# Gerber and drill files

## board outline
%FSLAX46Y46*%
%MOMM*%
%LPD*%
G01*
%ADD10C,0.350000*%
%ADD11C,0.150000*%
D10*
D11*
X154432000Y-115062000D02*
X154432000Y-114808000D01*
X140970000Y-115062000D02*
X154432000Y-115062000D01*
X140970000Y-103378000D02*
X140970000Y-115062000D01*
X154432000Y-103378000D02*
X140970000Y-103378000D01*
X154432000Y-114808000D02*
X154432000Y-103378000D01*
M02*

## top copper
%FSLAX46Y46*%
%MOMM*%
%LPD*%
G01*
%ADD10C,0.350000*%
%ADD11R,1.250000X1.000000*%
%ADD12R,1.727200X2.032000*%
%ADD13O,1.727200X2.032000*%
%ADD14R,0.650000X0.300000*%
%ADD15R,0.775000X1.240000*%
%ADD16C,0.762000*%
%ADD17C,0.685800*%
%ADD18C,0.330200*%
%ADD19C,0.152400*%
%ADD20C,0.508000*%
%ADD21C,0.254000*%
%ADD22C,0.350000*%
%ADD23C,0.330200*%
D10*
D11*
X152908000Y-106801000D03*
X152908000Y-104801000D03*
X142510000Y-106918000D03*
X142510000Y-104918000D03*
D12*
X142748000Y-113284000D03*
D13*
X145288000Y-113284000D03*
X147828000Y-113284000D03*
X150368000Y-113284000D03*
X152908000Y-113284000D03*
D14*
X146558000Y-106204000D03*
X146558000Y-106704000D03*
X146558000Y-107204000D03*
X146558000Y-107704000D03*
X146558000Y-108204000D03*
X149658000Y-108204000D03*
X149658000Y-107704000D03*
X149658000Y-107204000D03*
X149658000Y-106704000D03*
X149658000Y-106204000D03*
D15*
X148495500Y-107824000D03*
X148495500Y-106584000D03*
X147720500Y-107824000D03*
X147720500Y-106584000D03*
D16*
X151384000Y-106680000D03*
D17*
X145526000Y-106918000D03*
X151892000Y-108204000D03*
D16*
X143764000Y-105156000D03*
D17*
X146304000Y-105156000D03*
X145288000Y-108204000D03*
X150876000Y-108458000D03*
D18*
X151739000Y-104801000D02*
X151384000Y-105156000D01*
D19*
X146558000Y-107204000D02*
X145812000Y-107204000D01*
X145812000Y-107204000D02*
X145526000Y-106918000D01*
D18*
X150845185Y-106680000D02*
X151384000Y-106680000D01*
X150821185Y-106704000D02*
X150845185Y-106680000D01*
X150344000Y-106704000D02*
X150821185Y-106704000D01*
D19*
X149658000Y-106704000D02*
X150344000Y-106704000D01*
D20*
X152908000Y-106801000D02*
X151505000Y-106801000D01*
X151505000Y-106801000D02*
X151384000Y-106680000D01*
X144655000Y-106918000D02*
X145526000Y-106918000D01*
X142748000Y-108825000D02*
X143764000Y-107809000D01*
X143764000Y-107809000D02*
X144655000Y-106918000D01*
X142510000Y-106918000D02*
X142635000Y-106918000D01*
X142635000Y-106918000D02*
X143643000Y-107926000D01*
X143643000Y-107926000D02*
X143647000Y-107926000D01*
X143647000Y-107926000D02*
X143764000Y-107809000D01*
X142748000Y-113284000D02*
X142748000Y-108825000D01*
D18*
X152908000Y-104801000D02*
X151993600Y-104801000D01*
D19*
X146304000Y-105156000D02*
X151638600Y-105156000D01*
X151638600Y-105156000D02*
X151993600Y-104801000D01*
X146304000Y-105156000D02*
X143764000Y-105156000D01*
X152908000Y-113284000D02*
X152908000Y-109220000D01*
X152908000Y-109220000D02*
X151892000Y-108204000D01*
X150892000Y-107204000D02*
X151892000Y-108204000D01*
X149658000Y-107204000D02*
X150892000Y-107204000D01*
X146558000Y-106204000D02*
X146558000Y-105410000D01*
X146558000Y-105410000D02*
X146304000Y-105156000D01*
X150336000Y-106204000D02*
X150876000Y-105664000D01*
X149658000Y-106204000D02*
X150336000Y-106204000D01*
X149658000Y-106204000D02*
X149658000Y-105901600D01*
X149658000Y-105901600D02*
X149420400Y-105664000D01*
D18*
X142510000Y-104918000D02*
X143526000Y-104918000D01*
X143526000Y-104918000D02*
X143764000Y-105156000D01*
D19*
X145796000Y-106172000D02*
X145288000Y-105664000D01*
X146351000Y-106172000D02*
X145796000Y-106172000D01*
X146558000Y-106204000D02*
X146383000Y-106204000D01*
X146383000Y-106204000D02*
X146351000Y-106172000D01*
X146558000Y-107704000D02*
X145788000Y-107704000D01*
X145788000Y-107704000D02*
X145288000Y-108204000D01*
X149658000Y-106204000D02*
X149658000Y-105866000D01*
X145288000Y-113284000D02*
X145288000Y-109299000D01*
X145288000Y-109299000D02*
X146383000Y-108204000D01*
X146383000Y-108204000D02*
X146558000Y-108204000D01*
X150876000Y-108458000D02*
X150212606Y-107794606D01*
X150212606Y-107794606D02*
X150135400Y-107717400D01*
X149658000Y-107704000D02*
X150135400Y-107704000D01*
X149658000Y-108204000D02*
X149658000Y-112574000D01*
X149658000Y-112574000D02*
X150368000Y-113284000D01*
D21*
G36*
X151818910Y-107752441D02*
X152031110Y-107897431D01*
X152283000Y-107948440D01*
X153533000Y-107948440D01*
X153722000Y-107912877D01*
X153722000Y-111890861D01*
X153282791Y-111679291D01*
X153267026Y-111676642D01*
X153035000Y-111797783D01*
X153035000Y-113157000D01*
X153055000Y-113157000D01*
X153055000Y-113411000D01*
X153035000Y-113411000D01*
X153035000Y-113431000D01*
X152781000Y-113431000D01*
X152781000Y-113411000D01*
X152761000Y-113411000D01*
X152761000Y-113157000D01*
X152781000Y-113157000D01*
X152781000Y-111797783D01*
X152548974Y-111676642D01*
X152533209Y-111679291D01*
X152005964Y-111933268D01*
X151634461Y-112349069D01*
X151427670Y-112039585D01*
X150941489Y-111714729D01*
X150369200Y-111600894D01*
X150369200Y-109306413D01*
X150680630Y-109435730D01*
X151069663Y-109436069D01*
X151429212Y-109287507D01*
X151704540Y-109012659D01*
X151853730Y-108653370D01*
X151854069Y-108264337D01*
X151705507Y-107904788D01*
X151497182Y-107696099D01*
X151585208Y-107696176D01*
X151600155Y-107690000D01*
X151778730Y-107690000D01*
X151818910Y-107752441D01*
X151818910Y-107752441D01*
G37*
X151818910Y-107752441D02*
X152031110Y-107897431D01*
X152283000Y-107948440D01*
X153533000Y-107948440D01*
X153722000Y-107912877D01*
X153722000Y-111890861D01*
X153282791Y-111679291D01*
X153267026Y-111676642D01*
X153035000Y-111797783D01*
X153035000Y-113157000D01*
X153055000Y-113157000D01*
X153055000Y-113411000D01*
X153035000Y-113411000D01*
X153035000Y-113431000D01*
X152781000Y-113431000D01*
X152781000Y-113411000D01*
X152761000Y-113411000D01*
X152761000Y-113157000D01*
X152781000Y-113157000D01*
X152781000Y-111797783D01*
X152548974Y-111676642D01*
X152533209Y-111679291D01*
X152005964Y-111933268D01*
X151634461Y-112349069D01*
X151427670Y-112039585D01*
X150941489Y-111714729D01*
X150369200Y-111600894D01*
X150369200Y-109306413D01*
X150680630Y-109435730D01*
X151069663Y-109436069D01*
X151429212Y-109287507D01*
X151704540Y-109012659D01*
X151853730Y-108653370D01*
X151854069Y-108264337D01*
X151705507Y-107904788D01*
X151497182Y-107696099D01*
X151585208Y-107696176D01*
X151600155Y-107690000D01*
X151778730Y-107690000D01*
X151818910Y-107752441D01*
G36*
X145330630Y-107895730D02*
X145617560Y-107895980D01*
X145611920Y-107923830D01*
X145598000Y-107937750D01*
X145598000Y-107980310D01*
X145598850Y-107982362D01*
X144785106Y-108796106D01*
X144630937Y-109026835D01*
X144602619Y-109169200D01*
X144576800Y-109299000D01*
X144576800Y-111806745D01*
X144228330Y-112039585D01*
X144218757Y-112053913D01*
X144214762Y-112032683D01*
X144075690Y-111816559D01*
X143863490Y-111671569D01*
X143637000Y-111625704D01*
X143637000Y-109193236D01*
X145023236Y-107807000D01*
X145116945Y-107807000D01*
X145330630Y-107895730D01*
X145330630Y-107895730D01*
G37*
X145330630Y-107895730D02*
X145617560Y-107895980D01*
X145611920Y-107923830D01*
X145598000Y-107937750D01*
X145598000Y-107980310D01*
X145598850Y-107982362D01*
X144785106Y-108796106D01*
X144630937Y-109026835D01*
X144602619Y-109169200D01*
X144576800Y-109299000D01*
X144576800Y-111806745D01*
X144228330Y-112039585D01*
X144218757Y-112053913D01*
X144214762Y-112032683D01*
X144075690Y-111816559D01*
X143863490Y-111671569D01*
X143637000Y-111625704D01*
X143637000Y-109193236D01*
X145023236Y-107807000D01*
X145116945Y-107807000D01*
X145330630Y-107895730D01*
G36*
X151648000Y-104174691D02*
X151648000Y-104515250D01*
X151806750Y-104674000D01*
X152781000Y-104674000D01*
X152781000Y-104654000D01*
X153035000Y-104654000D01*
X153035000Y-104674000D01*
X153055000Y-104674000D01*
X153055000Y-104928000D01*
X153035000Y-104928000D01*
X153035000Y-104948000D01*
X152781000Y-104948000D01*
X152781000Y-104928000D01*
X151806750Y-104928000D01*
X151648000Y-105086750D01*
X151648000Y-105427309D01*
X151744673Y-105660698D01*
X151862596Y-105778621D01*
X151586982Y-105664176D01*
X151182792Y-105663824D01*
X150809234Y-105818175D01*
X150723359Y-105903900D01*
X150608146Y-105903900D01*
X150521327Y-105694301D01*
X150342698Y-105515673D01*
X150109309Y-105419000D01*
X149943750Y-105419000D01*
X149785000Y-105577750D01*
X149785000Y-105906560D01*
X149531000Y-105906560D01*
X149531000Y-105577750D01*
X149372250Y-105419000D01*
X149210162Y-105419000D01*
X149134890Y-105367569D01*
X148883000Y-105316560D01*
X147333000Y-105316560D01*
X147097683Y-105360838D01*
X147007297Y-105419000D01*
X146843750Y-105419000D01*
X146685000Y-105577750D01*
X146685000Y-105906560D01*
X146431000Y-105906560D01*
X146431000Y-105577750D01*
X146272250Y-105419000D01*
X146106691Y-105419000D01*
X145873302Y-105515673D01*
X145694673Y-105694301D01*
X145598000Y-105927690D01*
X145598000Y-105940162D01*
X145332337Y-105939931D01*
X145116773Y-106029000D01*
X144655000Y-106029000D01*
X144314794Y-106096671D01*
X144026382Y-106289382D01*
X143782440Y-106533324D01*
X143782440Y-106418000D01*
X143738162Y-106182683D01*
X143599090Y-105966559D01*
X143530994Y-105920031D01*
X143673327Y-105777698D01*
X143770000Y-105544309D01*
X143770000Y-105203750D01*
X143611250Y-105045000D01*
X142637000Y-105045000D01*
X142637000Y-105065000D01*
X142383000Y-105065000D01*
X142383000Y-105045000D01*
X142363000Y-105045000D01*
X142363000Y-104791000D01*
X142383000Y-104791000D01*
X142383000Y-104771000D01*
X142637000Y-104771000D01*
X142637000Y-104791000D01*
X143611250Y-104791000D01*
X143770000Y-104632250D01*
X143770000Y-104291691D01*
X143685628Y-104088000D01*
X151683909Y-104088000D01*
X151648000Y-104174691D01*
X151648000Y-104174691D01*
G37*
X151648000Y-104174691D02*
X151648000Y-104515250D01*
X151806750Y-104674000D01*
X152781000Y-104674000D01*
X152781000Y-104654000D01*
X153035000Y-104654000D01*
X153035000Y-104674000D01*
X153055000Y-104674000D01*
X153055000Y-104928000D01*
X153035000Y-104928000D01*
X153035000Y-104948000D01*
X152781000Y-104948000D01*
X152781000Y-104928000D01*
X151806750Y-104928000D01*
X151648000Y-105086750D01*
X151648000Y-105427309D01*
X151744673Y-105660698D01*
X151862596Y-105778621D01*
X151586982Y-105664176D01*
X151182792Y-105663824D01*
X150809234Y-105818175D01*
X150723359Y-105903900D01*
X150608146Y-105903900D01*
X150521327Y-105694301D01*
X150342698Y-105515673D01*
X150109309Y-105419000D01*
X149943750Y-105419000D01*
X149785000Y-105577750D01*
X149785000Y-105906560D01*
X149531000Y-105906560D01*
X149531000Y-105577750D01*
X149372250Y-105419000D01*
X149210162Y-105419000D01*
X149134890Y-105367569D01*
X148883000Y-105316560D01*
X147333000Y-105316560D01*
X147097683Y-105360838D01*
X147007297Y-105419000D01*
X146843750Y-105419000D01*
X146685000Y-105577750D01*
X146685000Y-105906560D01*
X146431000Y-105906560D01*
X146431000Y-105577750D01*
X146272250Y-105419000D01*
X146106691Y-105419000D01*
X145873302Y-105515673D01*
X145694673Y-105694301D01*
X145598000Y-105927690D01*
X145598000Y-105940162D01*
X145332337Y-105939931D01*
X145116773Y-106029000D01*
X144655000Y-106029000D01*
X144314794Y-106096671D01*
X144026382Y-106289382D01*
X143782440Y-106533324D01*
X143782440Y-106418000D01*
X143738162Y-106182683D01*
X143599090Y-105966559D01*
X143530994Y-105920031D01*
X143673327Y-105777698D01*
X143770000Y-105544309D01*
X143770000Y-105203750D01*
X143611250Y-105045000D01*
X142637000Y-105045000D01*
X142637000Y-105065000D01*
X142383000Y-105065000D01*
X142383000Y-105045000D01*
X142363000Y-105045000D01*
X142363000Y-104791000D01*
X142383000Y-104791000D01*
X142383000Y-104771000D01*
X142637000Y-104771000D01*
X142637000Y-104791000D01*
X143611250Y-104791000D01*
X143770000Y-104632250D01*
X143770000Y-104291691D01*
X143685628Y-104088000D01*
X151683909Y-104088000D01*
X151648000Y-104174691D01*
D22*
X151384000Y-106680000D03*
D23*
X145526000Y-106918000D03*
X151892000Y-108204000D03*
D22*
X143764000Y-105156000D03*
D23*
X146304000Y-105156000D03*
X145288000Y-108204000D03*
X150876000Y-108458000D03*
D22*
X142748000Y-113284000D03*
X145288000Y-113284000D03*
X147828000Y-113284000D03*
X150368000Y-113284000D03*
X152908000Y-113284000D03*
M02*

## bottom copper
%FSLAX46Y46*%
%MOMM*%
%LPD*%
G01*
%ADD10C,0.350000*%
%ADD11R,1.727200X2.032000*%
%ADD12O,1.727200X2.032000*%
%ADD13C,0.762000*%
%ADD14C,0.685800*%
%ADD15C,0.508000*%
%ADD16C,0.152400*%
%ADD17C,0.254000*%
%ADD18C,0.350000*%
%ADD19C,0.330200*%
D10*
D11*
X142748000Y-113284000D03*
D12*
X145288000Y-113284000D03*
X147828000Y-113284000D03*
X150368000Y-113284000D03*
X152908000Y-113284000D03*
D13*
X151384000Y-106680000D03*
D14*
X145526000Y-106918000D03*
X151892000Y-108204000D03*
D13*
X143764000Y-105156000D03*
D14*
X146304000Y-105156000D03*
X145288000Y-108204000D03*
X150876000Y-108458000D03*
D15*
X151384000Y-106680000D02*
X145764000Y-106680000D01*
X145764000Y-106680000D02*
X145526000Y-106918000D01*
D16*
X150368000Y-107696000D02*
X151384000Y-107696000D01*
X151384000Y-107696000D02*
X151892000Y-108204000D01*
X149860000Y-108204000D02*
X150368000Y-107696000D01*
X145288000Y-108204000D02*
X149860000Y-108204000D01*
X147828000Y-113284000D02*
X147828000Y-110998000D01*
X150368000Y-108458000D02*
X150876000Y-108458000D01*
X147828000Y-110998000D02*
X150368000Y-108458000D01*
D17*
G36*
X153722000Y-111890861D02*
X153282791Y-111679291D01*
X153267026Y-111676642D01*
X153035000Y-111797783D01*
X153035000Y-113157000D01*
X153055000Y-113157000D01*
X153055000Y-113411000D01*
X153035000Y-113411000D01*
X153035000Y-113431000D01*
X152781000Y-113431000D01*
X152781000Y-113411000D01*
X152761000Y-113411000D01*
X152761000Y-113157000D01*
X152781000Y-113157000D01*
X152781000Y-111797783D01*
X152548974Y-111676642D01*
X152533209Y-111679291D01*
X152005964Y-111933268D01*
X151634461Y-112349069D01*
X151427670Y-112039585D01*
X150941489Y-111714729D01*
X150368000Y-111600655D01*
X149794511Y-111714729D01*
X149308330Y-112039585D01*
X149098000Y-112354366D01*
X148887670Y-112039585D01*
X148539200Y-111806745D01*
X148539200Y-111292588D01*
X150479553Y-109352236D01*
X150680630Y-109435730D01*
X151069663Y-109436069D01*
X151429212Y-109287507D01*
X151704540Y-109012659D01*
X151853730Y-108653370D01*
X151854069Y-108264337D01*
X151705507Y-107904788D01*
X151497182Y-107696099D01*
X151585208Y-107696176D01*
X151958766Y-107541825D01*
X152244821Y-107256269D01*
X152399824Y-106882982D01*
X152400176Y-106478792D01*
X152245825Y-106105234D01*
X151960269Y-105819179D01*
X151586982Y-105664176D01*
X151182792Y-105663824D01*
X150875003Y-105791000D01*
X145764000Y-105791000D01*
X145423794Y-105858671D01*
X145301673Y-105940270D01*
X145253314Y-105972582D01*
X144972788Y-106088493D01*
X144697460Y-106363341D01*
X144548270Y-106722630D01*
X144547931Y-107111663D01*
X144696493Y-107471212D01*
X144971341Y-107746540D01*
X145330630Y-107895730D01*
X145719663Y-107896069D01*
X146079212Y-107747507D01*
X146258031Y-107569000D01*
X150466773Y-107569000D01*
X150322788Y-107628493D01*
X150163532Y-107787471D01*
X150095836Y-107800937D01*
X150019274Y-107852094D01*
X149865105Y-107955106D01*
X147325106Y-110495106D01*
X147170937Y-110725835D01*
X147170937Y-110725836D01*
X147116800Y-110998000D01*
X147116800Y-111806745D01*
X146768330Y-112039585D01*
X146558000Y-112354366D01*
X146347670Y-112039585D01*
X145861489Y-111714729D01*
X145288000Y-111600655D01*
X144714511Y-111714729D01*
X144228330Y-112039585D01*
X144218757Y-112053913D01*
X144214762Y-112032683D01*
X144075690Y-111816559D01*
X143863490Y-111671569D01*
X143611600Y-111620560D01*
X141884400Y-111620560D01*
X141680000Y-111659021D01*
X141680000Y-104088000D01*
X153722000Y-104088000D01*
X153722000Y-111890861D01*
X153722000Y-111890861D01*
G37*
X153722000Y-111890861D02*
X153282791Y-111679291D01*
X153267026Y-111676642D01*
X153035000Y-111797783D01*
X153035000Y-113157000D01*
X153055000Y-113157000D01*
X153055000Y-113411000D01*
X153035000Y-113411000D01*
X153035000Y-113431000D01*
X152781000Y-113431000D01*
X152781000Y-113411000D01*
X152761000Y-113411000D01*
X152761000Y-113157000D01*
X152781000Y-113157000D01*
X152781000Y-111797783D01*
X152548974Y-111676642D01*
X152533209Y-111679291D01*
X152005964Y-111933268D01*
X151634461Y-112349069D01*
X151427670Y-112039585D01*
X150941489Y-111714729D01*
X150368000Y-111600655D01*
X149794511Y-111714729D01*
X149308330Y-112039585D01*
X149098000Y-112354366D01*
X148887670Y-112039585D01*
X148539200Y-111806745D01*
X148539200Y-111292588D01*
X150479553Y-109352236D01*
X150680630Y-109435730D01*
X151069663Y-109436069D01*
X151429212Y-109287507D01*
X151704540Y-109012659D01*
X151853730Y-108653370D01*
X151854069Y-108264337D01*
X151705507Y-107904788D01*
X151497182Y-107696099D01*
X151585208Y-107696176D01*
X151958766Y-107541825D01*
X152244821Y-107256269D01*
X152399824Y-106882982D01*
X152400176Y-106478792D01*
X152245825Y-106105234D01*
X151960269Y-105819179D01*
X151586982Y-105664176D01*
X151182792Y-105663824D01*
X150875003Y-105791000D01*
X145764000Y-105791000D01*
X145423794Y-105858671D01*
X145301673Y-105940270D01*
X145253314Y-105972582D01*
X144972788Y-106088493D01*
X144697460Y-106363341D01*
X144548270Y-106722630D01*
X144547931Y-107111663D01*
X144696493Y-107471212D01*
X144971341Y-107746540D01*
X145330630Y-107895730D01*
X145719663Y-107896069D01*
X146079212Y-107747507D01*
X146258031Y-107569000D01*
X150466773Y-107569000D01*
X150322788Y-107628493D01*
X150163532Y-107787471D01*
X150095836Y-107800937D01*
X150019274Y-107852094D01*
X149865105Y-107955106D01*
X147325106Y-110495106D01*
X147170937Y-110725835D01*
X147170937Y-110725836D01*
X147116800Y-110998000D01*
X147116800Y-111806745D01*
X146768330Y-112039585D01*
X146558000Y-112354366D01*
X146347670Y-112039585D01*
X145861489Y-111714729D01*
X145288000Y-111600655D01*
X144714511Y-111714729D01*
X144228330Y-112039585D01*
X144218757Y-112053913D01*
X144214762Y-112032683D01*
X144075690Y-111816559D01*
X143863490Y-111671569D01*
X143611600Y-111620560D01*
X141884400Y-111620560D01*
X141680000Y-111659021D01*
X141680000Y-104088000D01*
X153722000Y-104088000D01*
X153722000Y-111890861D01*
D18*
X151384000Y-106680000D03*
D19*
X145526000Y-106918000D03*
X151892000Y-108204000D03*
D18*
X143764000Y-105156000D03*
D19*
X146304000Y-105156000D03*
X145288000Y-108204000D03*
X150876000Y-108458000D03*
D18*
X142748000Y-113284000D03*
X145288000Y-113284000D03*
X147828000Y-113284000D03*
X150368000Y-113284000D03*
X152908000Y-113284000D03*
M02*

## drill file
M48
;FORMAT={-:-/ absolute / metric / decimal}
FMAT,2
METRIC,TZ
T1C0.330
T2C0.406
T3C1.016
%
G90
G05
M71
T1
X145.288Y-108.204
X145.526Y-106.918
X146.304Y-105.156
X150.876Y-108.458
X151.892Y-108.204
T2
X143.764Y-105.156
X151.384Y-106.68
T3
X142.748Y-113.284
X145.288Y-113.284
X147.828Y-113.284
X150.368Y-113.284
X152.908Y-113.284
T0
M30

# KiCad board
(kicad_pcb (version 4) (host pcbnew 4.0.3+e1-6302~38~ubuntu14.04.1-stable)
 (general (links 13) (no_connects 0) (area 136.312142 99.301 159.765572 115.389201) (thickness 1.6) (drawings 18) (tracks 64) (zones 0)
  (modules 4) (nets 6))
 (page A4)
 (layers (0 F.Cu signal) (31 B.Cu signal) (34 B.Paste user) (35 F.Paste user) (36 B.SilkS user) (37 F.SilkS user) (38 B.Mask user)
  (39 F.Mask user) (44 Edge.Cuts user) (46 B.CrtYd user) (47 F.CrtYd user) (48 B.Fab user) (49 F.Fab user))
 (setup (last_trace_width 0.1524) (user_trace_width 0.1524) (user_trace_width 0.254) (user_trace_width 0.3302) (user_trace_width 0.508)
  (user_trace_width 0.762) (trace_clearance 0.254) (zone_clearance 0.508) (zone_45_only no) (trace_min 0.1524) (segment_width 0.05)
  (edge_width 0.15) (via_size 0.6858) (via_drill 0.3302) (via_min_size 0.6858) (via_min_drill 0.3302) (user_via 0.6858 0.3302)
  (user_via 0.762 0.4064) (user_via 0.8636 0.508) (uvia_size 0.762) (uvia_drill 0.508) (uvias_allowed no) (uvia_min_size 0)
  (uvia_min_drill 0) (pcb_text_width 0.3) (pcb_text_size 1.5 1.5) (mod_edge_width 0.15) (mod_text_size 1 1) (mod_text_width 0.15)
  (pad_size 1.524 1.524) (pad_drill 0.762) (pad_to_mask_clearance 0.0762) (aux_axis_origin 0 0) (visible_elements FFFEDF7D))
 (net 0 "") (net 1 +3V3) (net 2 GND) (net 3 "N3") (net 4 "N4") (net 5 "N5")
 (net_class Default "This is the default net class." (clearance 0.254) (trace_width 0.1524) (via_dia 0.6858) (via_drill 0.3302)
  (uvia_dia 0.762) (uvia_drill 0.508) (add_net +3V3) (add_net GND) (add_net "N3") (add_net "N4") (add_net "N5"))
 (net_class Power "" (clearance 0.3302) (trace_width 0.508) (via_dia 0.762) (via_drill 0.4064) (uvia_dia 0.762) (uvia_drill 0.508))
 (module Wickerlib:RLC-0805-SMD (layer F.Cu) (at 152.908 105.801 90)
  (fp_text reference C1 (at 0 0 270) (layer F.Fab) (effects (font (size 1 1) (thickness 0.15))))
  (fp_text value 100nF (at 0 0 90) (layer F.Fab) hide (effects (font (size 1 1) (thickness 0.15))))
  (pad 1 smd rect (at -1 0 90) (size 1 1.25) (layers F.Cu F.Paste F.Mask) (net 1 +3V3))
  (pad 2 smd rect (at 1 0 90) (size 1 1.25) (layers F.Cu F.Paste F.Mask) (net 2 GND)))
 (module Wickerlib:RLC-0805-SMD (layer F.Cu) (at 142.51 105.918 90)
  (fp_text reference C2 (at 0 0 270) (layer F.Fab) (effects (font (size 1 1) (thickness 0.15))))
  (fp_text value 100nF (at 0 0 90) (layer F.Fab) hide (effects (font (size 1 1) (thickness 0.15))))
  (pad 1 smd rect (at -1 0 90) (size 1 1.25) (layers F.Cu F.Paste F.Mask) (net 1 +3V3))
  (pad 2 smd rect (at 1 0 90) (size 1 1.25) (layers F.Cu F.Paste F.Mask) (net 2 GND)))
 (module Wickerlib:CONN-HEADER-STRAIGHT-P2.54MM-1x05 (layer F.Cu) (at 142.748 113.284 90)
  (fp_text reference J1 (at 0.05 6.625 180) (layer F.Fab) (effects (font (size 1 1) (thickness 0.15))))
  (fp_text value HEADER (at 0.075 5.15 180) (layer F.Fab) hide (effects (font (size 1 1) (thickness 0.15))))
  (pad 1 thru_hole rect (at 0 0 90) (size 2.032 1.7272) (drill 1.016) (layers *.Cu *.Mask F.SilkS) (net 1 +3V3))
  (pad 2 thru_hole oval (at 0 2.54 90) (size 2.032 1.7272) (drill 1.016) (layers *.Cu *.Mask F.SilkS) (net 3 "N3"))
  (pad 3 thru_hole oval (at 0 5.08 90) (size 2.032 1.7272) (drill 1.016) (layers *.Cu *.Mask F.SilkS) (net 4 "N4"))
  (pad 4 thru_hole oval (at 0 7.62 90) (size 2.032 1.7272) (drill 1.016) (layers *.Cu *.Mask F.SilkS) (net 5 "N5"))
  (pad 5 thru_hole oval (at 0 10.16 90) (size 2.032 1.7272) (drill 1.016) (layers *.Cu *.Mask F.SilkS) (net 2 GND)))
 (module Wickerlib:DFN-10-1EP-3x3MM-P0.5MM (layer F.Cu) (at 148.108 107.204)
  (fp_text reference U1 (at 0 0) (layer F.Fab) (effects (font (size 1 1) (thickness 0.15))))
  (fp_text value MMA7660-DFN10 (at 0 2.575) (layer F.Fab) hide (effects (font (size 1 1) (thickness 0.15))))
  (pad 1 smd rect (at -1.55 -1) (size 0.65 0.3) (layers F.Cu F.Paste F.Mask) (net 2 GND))
  (pad 2 smd rect (at -1.55 -0.5) (size 0.65 0.3) (layers F.Cu F.Paste F.Mask))
  (pad 3 smd rect (at -1.55 0) (size 0.65 0.3) (layers F.Cu F.Paste F.Mask) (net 1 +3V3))
  (pad 4 smd rect (at -1.55 0.5) (size 0.65 0.3) (layers F.Cu F.Paste F.Mask) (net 2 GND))
  (pad 5 smd rect (at -1.55 1) (size 0.65 0.3) (layers F.Cu F.Paste F.Mask) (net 3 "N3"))
  (pad 6 smd rect (at 1.55 1) (size 0.65 0.3) (layers F.Cu F.Paste F.Mask) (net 5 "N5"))
  (pad 7 smd rect (at 1.55 0.5) (size 0.65 0.3) (layers F.Cu F.Paste F.Mask) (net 4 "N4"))
  (pad 8 smd rect (at 1.55 0) (size 0.65 0.3) (layers F.Cu F.Paste F.Mask) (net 2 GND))
  (pad 9 smd rect (at 1.55 -0.5) (size 0.65 0.3) (layers F.Cu F.Paste F.Mask) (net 1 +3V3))
  (pad 10 smd rect (at 1.55 -1) (size 0.65 0.3) (layers F.Cu F.Paste F.Mask) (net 2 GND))
  (pad 11 smd rect (at 0.3875 0.62) (size 0.775 1.24) (layers F.Cu F.Paste F.Mask) (solder_paste_margin_ratio -0.2))
  (pad 11 smd rect (at 0.3875 -0.62) (size 0.775 1.24) (layers F.Cu F.Paste F.Mask) (solder_paste_margin_ratio -0.2))
  (pad 11 smd rect (at -0.3875 0.62) (size 0.775 1.24) (layers F.Cu F.Paste F.Mask) (solder_paste_margin_ratio -0.2))
  (pad 11 smd rect (at -0.3875 -0.62) (size 0.775 1.24) (layers F.Cu F.Paste F.Mask) (solder_paste_margin_ratio -0.2)))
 (gr_line (start 154.432 115.062) (end 154.432 114.808) (layer Edge.Cuts) (width 0.15))
 (gr_line (start 140.97 115.062) (end 154.432 115.062) (layer Edge.Cuts) (width 0.15))
 (gr_line (start 140.97 103.378) (end 140.97 115.062) (layer Edge.Cuts) (width 0.15))
 (gr_line (start 154.432 103.378) (end 140.97 103.378) (layer Edge.Cuts) (width 0.15))
 (gr_line (start 154.432 114.808) (end 154.432 103.378) (layer Edge.Cuts) (width 0.15))
 (segment (start 151.739 104.801) (end 151.384 105.156) (width 0.3302) (layer F.Cu) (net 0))
 (segment (start 146.558 107.204) (end 145.812 107.204) (width 0.1524) (layer F.Cu) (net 1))
 (segment (start 145.812 107.204) (end 145.526 106.918) (width 0.1524) (layer F.Cu) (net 1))
 (segment (start 150.845185 106.68) (end 151.384 106.68) (width 0.3302) (layer F.Cu) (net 1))
 (segment (start 150.821185 106.704) (end 150.845185 106.68) (width 0.3302) (layer F.Cu) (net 1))
 (segment (start 150.344 106.704) (end 150.821185 106.704) (width 0.3302) (layer F.Cu) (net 1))
 (segment (start 149.658 106.704) (end 150.344 106.704) (width 0.1524) (layer F.Cu) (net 1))
 (segment (start 151.384 106.68) (end 145.764 106.68) (width 0.508) (layer B.Cu) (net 1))
 (segment (start 145.764 106.68) (end 145.526 106.918) (width 0.508) (layer B.Cu) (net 1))
 (segment (start 152.908 106.801) (end 151.505 106.801) (width 0.508) (layer F.Cu) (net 1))
 (segment (start 151.505 106.801) (end 151.384 106.68) (width 0.508) (layer F.Cu) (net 1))
 (via (at 151.384 106.68) (size 0.762) (drill 0.4064) (layers F.Cu B.Cu) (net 1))
 (via (at 145.526 106.918) (size 0.6858) (drill 0.3302) (layers F.Cu B.Cu) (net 1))
 (segment (start 144.655 106.918) (end 145.526 106.918) (width 0.508) (layer F.Cu) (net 1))
 (segment (start 142.748 108.825) (end 143.764 107.809) (width 0.508) (layer F.Cu) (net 1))
 (segment (start 143.764 107.809) (end 144.655 106.918) (width 0.508) (layer F.Cu) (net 1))
 (segment (start 142.51 106.918) (end 142.635 106.918) (width 0.508) (layer F.Cu) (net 1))
 (segment (start 142.635 106.918) (end 143.643 107.926) (width 0.508) (layer F.Cu) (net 1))
 (segment (start 143.643 107.926) (end 143.647 107.926) (width 0.508) (layer F.Cu) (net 1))
 (segment (start 143.647 107.926) (end 143.764 107.809) (width 0.508) (layer F.Cu) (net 1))
 (segment (start 142.748 113.284) (end 142.748 108.825) (width 0.508) (layer F.Cu) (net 1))
 (segment (start 152.908 104.801) (end 151.9936 104.801) (width 0.3302) (layer F.Cu) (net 2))
 (segment (start 146.304 105.156) (end 151.6386 105.156) (width 0.1524) (layer F.Cu) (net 2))
 (segment (start 151.6386 105.156) (end 151.9936 104.801) (width 0.1524) (layer F.Cu) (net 2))
 (segment (start 146.304 105.156) (end 143.764 105.156) (width 0.1524) (layer F.Cu) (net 2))
 (segment (start 152.908 113.284) (end 152.908 109.22) (width 0.1524) (layer F.Cu) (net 2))
 (segment (start 152.908 109.22) (end 151.892 108.204) (width 0.1524) (layer F.Cu) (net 2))
 (segment (start 150.368 107.696) (end 151.384 107.696) (width 0.1524) (layer B.Cu) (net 2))
 (segment (start 151.384 107.696) (end 151.892 108.204) (width 0.1524) (layer B.Cu) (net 2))
 (via (at 151.892 108.204) (size 0.6858) (drill 0.3302) (layers F.Cu B.Cu) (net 2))
 (segment (start 149.86 108.204) (end 150.368 107.696) (width 0.1524) (layer B.Cu) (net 2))
 (segment (start 145.288 108.204) (end 149.86 108.204) (width 0.1524) (layer B.Cu) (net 2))
 (segment (start 150.892 107.204) (end 151.892 108.204) (width 0.1524) (layer F.Cu) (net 2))
 (segment (start 149.658 107.204) (end 150.892 107.204) (width 0.1524) (layer F.Cu) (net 2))
 (segment (start 146.558 106.204) (end 146.558 105.41) (width 0.1524) (layer F.Cu) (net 2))
 (segment (start 146.558 105.41) (end 146.304 105.156) (width 0.1524) (layer F.Cu) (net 2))
 (segment (start 150.336 106.204) (end 150.876 105.664) (width 0.1524) (layer F.Cu) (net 2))
 (segment (start 149.658 106.204) (end 150.336 106.204) (width 0.1524) (layer F.Cu) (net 2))
 (segment (start 149.658 106.204) (end 149.658 105.9016) (width 0.1524) (layer F.Cu) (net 2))
 (segment (start 149.658 105.9016) (end 149.4204 105.664) (width 0.1524) (layer F.Cu) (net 2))
 (segment (start 142.51 104.918) (end 143.526 104.918) (width 0.3302) (layer F.Cu) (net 2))
 (via (at 143.764 105.156) (size 0.762) (drill 0.4064) (layers F.Cu B.Cu) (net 2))
 (segment (start 143.526 104.918) (end 143.764 105.156) (width 0.3302) (layer F.Cu) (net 2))
 (segment (start 145.796 106.172) (end 145.288 105.664) (width 0.1524) (layer F.Cu) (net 2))
 (segment (start 146.351 106.172) (end 145.796 106.172) (width 0.1524) (layer F.Cu) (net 2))
 (segment (start 146.558 106.204) (end 146.383 106.204) (width 0.1524) (layer F.Cu) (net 2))
 (segment (start 146.383 106.204) (end 146.351 106.172) (width 0.1524) (layer F.Cu) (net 2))
 (via (at 146.304 105.156) (size 0.6858) (drill 0.3302) (layers F.Cu B.Cu) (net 2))
 (segment (start 146.558 107.704) (end 145.788 107.704) (width 0.1524) (layer F.Cu) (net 2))
 (segment (start 145.788 107.704) (end 145.288 108.204) (width 0.1524) (layer F.Cu) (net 2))
 (via (at 145.288 108.204) (size 0.6858) (drill 0.3302) (layers F.Cu B.Cu) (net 2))
 (segment (start 149.658 106.204) (end 149.658 105.866) (width 0.1524) (layer F.Cu) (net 2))
 (segment (start 145.288 113.284) (end 145.288 109.299) (width 0.1524) (layer F.Cu) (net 3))
 (segment (start 145.288 109.299) (end 146.383 108.204) (width 0.1524) (layer F.Cu) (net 3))
 (segment (start 146.383 108.204) (end 146.558 108.204) (width 0.1524) (layer F.Cu) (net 3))
 (via (at 150.876 108.458) (size 0.6858) (drill 0.3302) (layers F.Cu B.Cu) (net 4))
 (segment (start 150.876 108.458) (end 150.212606 107.794606) (width 0.1524) (layer F.Cu) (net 4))
 (segment (start 150.212606 107.794606) (end 150.1354 107.7174) (width 0.1524) (layer F.Cu) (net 4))
 (segment (start 147.828 113.284) (end 147.828 110.998) (width 0.1524) (layer B.Cu) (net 4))
 (segment (start 150.368 108.458) (end 150.876 108.458) (width 0.1524) (layer B.Cu) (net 4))
 (segment (start 147.828 110.998) (end 150.368 108.458) (width 0.1524) (layer B.Cu) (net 4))
 (segment (start 149.658 107.704) (end 150.1354 107.704) (width 0.1524) (layer F.Cu) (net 4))
 (segment (start 149.658 108.204) (end 149.658 112.574) (width 0.1524) (layer F.Cu) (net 5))
 (segment (start 149.658 112.574) (end 150.368 113.284) (width 0.1524) (layer F.Cu) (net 5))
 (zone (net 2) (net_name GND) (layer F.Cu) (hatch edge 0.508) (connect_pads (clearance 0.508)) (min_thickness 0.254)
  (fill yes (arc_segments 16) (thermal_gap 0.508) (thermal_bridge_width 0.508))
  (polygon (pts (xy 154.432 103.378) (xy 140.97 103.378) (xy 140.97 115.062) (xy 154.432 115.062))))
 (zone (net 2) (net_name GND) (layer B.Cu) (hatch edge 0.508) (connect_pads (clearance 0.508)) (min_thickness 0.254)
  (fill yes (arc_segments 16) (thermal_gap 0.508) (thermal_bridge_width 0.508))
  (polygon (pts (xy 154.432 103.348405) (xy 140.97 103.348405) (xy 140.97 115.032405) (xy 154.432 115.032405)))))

